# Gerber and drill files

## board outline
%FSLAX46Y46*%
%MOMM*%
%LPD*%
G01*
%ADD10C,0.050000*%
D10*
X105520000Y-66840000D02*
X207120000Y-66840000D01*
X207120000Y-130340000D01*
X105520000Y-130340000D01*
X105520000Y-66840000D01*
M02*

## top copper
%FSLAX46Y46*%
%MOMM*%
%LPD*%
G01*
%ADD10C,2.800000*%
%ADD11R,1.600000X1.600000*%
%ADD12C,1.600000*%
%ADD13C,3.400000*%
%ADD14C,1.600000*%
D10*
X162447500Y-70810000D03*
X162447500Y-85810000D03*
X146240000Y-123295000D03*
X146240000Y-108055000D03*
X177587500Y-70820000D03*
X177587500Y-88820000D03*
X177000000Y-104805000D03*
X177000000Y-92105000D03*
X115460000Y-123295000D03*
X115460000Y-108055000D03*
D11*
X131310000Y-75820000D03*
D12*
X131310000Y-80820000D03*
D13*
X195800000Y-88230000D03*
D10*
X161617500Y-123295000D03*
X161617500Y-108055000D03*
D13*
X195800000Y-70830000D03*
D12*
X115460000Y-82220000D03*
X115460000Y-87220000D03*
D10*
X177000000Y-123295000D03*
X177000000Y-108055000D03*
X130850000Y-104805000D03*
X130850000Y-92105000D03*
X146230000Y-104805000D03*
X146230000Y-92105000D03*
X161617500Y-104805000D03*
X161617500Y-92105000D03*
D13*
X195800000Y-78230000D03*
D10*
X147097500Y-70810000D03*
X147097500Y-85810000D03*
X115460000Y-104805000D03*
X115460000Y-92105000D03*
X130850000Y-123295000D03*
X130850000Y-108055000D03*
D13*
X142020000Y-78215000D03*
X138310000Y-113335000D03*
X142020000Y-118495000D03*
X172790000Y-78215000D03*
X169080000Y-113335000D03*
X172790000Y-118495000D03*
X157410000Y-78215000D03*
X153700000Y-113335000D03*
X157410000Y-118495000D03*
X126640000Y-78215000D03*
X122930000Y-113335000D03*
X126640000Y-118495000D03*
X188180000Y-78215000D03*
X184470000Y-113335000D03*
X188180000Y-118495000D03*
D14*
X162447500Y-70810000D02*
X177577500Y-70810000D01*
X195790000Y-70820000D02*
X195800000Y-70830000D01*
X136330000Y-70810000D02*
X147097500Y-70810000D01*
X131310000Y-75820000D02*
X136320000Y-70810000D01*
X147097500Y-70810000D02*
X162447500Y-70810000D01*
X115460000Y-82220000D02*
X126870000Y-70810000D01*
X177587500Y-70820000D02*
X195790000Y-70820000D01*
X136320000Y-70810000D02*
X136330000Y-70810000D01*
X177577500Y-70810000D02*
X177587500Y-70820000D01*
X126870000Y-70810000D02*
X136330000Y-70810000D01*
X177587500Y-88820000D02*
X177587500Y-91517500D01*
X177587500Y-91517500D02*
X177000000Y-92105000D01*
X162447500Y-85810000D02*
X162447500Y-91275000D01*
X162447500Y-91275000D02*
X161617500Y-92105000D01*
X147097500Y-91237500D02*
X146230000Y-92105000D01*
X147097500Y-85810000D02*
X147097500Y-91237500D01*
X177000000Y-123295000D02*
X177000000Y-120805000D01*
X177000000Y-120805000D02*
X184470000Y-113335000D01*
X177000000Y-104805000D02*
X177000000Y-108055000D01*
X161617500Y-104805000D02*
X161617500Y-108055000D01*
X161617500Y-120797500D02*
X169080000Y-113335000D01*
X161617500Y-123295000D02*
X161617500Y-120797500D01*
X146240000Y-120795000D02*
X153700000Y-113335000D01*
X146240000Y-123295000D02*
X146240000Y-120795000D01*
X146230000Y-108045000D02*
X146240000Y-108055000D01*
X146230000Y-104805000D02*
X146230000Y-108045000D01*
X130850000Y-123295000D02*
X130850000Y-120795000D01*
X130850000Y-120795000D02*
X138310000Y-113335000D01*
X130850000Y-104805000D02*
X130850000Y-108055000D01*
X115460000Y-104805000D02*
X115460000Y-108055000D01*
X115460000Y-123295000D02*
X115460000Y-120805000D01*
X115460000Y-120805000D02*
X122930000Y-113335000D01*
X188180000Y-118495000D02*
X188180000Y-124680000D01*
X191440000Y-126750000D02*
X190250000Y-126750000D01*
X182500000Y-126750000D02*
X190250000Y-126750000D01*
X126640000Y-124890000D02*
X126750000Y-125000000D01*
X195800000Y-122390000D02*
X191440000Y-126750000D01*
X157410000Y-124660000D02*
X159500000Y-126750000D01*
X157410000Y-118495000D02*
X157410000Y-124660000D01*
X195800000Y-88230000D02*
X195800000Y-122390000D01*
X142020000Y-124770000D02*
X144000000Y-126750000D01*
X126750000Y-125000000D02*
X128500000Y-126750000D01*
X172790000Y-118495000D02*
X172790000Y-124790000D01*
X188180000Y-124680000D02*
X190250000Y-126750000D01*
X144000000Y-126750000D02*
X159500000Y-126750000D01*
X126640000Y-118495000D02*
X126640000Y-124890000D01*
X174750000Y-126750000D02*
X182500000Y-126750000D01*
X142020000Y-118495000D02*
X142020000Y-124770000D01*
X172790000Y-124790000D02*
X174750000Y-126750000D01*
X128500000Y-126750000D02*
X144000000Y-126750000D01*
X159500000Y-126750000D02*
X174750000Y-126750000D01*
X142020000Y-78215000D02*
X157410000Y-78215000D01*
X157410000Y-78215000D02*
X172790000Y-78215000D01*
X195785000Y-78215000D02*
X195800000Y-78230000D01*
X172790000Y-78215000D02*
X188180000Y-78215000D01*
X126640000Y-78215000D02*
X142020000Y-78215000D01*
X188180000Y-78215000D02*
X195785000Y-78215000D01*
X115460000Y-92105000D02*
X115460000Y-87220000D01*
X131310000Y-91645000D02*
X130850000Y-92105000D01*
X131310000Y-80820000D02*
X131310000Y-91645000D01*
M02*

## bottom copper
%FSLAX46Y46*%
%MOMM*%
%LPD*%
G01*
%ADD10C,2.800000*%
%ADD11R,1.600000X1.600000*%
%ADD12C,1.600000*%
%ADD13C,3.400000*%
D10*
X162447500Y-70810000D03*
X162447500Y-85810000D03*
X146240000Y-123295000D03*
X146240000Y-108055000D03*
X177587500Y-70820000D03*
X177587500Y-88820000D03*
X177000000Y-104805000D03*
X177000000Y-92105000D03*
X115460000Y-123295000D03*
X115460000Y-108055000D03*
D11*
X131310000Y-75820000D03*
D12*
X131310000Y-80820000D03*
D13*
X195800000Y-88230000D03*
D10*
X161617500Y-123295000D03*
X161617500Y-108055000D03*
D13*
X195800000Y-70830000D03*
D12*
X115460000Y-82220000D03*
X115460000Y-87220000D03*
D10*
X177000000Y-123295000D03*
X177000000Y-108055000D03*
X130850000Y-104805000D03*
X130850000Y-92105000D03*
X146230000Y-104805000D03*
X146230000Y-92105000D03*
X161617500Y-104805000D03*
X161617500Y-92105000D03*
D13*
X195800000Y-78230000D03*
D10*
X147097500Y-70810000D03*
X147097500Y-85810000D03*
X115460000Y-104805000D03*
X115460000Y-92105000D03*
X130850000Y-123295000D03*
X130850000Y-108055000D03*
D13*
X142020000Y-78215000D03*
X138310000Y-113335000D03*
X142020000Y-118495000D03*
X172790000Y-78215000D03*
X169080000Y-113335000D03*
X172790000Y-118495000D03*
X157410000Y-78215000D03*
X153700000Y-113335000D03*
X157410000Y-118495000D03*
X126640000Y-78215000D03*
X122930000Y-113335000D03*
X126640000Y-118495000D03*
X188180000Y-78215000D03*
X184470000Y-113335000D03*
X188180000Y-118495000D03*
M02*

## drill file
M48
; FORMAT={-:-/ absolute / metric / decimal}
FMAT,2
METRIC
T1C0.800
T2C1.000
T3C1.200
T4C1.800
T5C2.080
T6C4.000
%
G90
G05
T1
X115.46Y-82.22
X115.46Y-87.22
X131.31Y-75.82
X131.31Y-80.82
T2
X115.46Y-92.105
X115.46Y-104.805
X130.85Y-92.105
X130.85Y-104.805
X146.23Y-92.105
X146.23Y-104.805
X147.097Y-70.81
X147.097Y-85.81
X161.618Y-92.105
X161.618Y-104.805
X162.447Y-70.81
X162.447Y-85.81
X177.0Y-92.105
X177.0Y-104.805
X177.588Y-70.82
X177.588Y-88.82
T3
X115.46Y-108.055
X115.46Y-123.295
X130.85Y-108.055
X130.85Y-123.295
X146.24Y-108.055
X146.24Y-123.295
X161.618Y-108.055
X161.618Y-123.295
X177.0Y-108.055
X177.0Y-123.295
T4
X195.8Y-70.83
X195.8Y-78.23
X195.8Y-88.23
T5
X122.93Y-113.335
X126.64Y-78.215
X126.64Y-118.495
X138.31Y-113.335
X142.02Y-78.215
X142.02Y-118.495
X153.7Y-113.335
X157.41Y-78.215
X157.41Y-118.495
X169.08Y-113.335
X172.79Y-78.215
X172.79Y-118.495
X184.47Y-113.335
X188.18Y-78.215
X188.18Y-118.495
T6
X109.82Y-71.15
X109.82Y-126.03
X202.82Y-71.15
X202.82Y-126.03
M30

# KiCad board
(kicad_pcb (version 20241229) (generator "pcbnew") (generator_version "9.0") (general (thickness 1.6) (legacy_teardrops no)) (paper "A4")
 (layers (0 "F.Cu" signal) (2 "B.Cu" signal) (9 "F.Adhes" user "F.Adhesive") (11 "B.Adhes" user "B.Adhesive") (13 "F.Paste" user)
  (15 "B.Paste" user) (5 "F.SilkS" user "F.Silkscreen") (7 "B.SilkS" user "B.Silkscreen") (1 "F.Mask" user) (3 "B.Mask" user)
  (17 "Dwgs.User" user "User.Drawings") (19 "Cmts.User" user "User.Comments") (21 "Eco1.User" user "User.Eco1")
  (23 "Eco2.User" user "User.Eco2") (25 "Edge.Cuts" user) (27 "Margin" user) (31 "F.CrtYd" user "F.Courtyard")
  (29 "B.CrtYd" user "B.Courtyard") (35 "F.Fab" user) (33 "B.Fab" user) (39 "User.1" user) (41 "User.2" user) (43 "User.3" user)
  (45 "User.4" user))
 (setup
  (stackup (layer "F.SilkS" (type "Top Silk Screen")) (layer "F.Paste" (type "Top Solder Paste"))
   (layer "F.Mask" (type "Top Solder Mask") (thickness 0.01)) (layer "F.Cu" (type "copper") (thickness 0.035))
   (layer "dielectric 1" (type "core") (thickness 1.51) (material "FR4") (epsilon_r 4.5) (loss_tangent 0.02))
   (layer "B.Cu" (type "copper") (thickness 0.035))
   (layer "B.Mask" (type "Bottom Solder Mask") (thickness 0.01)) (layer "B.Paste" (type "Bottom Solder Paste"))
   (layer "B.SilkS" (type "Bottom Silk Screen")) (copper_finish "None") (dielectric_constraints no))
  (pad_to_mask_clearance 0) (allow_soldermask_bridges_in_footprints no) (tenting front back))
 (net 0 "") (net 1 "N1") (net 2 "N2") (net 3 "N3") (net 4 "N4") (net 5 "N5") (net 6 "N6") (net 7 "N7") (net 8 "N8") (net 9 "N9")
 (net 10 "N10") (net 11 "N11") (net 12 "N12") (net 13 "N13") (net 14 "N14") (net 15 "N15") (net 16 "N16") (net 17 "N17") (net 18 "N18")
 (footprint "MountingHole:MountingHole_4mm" (layer "F.Cu") (at 202.82 126.03)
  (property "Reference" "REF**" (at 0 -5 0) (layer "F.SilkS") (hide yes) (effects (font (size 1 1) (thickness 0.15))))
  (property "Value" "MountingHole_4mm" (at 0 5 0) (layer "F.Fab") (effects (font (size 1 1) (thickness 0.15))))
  (pad "" np_thru_hole circle (at 0 0) (size 4 4) (drill 4) (layers "*.Cu" "*.Mask")))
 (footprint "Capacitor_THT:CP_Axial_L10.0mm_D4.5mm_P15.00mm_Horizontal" (layer "F.Cu") (at 162.4475 70.81 -90)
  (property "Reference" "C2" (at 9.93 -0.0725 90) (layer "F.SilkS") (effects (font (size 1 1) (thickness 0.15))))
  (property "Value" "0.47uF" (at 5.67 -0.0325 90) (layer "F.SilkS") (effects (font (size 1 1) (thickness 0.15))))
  (pad "1" thru_hole circle (at 0 0 270) (size 2.8 2.8) (drill 1) (layers "*.Cu" "*.Mask") (remove_unused_layers no) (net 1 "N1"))
  (pad "2" thru_hole circle (at 15 0 270) (size 2.8 2.8) (drill 1) (layers "*.Cu" "*.Mask") (remove_unused_layers no) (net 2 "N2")))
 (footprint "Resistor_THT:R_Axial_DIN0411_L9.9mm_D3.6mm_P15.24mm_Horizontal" (layer "F.Cu") (at 146.24 123.295 90)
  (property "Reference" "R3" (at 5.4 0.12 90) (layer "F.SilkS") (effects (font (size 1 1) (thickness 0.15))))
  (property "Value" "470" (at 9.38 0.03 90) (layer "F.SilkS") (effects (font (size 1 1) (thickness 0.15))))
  (pad "1" thru_hole circle (at 0 0 90) (size 2.8 2.8) (drill 1.2) (layers "*.Cu" "*.Mask") (remove_unused_layers no) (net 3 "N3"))
  (pad "2" thru_hole circle (at 15.24 0 90) (size 2.8 2.8) (drill 1.2) (layers "*.Cu" "*.Mask") (remove_unused_layers no) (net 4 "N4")))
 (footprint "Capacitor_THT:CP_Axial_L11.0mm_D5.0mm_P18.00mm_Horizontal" (layer "F.Cu") (at 177.5875 70.82 -90)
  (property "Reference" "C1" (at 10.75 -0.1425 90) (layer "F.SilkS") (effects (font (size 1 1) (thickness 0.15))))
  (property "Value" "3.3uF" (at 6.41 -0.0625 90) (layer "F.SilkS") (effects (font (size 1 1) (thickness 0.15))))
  (pad "1" thru_hole circle (at 0 0 270) (size 2.8 2.8) (drill 1) (layers "*.Cu" "*.Mask") (remove_unused_layers no) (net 1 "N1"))
  (pad "2" thru_hole circle (at 18 0 270) (size 2.8 2.8) (drill 1) (layers "*.Cu" "*.Mask") (remove_unused_layers no) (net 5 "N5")))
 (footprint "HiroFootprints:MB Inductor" (layer "F.Cu") (at 177 104.805 90)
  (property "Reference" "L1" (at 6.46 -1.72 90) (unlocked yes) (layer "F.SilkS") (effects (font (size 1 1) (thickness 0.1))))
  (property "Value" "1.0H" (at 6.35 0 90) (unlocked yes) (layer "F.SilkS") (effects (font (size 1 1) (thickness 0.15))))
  (pad "1" thru_hole circle (at 0 0 90) (size 2.8 2.8) (drill 1) (layers "*.Cu" "*.Mask") (remove_unused_layers no) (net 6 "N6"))
  (pad "2" thru_hole circle (at 12.7 0 90) (size 2.8 2.8) (drill 1) (layers "*.Cu" "*.Mask") (remove_unused_layers no) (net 5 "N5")))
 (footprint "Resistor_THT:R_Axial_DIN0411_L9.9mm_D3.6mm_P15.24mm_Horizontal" (layer "F.Cu") (at 115.46 123.295 90)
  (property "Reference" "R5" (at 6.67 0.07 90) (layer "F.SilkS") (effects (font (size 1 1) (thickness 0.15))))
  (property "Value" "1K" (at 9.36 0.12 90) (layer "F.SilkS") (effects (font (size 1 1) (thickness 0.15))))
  (pad "1" thru_hole circle (at 0 0 90) (size 2.8 2.8) (drill 1.2) (layers "*.Cu" "*.Mask") (remove_unused_layers no) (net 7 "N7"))
  (pad "2" thru_hole circle (at 15.24 0 90) (size 2.8 2.8) (drill 1.2) (layers "*.Cu" "*.Mask") (remove_unused_layers no) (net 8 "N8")))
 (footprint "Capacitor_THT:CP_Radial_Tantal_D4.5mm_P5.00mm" (layer "F.Cu") (at 131.31 75.82 -90)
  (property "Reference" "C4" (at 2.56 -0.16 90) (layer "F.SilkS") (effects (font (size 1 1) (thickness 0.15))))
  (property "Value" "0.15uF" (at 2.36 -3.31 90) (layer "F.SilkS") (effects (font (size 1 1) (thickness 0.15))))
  (pad "1" thru_hole rect (at 0 0 270) (size 1.6 1.6) (drill 0.8) (layers "*.Cu" "*.Mask") (remove_unused_layers no) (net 1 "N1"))
  (pad "2" thru_hole circle (at 5 0 270) (size 1.6 1.6) (drill 0.8) (layers "*.Cu" "*.Mask") (remove_unused_layers no) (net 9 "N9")))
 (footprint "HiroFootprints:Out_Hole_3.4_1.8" (layer "F.Cu") (at 195.8 88.23)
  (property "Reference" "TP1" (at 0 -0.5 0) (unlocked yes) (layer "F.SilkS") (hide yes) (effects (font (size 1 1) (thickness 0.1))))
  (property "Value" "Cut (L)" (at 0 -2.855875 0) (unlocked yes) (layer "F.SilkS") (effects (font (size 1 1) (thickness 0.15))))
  (pad "1" thru_hole circle (at 0 0) (size 3.4 3.4) (drill 1.8) (layers "*.Cu" "*.Mask") (remove_unused_layers no) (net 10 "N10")))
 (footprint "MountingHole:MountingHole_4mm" (layer "F.Cu") (at 109.82 71.15)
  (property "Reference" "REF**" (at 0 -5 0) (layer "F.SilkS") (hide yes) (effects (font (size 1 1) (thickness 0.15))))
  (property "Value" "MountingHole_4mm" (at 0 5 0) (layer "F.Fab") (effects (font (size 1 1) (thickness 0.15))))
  (pad "" np_thru_hole circle (at 0 0) (size 4 4) (drill 4) (layers "*.Cu" "*.Mask")))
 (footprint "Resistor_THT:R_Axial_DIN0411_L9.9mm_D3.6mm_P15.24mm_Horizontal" (layer "F.Cu") (at 161.6175 123.295 90)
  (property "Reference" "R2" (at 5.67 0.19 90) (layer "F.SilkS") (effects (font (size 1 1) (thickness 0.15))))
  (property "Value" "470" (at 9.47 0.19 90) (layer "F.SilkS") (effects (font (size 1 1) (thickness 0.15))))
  (pad "1" thru_hole circle (at 0 0 90) (size 2.8 2.8) (drill 1.2) (layers "*.Cu" "*.Mask") (remove_unused_layers no) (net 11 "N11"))
  (pad "2" thru_hole circle (at 15.24 0 90) (size 2.8 2.8) (drill 1.2) (layers "*.Cu" "*.Mask") (remove_unused_layers no) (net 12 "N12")))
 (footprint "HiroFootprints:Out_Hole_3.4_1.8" (layer "F.Cu") (at 195.8 70.83)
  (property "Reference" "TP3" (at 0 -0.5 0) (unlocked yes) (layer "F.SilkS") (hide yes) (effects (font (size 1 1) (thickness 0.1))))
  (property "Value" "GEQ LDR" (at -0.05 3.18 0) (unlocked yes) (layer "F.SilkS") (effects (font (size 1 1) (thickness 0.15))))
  (pad "1" thru_hole circle (at 0 0) (size 3.4 3.4) (drill 1.8) (layers "*.Cu" "*.Mask") (remove_unused_layers no) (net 1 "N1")))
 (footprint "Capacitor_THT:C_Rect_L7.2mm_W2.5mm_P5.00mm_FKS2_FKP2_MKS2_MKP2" (layer "F.Cu") (at 115.46 82.22 -90)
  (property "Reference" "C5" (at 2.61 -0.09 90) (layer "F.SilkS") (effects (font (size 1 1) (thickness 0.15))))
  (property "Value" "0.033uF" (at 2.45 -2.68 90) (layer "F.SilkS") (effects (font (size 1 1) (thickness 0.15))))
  (pad "1" thru_hole circle (at 0 0 270) (size 1.6 1.6) (drill 0.8) (layers "*.Cu" "*.Mask") (remove_unused_layers no) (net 1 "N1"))
  (pad "2" thru_hole circle (at 5 0 270) (size 1.6 1.6) (drill 0.8) (layers "*.Cu" "*.Mask") (remove_unused_layers no) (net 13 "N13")))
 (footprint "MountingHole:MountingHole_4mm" (layer "F.Cu") (at 202.82 71.15)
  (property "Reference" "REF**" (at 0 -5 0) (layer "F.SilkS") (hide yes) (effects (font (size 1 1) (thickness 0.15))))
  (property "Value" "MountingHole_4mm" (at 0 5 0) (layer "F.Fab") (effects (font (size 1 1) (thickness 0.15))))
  (pad "" np_thru_hole circle (at 0 0) (size 4 4) (drill 4) (layers "*.Cu" "*.Mask")))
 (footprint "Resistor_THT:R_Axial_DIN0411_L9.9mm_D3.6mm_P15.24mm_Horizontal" (layer "F.Cu") (at 177 123.295 90)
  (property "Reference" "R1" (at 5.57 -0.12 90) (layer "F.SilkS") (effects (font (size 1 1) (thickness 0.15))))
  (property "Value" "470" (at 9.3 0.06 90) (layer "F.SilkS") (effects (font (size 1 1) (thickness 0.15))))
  (pad "1" thru_hole circle (at 0 0 90) (size 2.8 2.8) (drill 1.2) (layers "*.Cu" "*.Mask") (remove_unused_layers no) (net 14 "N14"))
  (pad "2" thru_hole circle (at 15.24 0 90) (size 2.8 2.8) (drill 1.2) (layers "*.Cu" "*.Mask") (remove_unused_layers no) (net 6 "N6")))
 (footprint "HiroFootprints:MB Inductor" (layer "F.Cu") (at 130.85 104.805 90)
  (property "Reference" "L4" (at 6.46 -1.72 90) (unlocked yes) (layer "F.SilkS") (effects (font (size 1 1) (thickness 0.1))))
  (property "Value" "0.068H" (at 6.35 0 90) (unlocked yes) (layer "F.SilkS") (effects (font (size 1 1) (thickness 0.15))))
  (pad "1" thru_hole circle (at 0 0 90) (size 2.8 2.8) (drill 1) (layers "*.Cu" "*.Mask") (remove_unused_layers no) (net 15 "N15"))
  (pad "2" thru_hole circle (at 12.7 0 90) (size 2.8 2.8) (drill 1) (layers "*.Cu" "*.Mask") (remove_unused_layers no) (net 9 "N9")))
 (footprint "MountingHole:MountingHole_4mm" (layer "F.Cu") (at 109.82 126.03)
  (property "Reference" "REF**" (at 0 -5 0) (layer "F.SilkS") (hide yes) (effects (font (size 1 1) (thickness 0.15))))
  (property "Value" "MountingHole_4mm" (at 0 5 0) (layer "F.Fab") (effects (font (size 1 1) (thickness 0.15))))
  (pad "" np_thru_hole circle (at 0 0) (size 4 4) (drill 4) (layers "*.Cu" "*.Mask")))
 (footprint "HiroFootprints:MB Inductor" (layer "F.Cu") (at 146.23 104.805 90)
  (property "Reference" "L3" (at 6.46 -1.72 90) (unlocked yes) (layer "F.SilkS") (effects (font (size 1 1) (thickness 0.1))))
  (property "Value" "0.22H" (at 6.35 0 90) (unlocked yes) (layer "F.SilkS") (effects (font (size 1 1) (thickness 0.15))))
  (pad "1" thru_hole circle (at 0 0 90) (size 2.8 2.8) (drill 1) (layers "*.Cu" "*.Mask") (remove_unused_layers no) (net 4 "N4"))
  (pad "2" thru_hole circle (at 12.7 0 90) (size 2.8 2.8) (drill 1) (layers "*.Cu" "*.Mask") (remove_unused_layers no) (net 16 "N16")))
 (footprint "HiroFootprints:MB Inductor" (layer "F.Cu") (at 161.6175 104.805 90)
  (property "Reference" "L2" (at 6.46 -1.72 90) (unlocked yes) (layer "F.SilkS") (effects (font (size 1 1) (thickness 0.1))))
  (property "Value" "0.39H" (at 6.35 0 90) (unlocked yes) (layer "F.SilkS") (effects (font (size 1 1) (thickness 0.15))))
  (pad "1" thru_hole circle (at 0 0 90) (size 2.8 2.8) (drill 1) (layers "*.Cu" "*.Mask") (remove_unused_layers no) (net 12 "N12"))
  (pad "2" thru_hole circle (at 12.7 0 90) (size 2.8 2.8) (drill 1) (layers "*.Cu" "*.Mask") (remove_unused_layers no) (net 2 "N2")))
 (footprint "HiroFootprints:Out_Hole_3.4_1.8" (layer "F.Cu") (at 195.8 78.23)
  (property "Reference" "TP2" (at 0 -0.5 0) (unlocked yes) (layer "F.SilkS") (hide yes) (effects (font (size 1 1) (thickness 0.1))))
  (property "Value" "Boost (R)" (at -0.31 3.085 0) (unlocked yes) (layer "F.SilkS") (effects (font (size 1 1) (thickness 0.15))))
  (pad "1" thru_hole circle (at 0 0) (size 3.4 3.4) (drill 1.8) (layers "*.Cu" "*.Mask") (remove_unused_layers no) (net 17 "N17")))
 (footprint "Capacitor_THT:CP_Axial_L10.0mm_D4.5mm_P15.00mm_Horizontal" (layer "F.Cu") (at 147.0975 70.81 -90)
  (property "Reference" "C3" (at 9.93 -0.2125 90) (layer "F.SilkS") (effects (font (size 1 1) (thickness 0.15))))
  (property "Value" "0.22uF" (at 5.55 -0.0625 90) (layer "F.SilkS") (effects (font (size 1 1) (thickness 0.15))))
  (pad "1" thru_hole circle (at 0 0 270) (size 2.8 2.8) (drill 1) (layers "*.Cu" "*.Mask") (remove_unused_layers no) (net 1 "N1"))
  (pad "2" thru_hole circle (at 15 0 270) (size 2.8 2.8) (drill 1) (layers "*.Cu" "*.Mask") (remove_unused_layers no) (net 16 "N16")))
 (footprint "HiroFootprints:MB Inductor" (layer "F.Cu") (at 115.46 104.805 90)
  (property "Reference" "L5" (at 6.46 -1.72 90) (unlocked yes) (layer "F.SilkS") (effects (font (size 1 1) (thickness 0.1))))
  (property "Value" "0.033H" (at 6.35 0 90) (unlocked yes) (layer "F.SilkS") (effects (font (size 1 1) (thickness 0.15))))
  (pad "1" thru_hole circle (at 0 0 90) (size 2.8 2.8) (drill 1) (layers "*.Cu" "*.Mask") (remove_unused_layers no) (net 8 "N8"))
  (pad "2" thru_hole circle (at 12.7 0 90) (size 2.8 2.8) (drill 1) (layers "*.Cu" "*.Mask") (remove_unused_layers no) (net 13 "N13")))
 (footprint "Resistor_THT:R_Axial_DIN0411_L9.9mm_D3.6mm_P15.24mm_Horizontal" (layer "F.Cu") (at 130.85 123.295 90)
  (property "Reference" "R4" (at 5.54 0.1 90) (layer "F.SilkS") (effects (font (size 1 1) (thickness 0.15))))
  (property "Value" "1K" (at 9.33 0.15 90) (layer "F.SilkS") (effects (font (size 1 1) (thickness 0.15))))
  (pad "1" thru_hole circle (at 0 0 90) (size 2.8 2.8) (drill 1.2) (layers "*.Cu" "*.Mask") (remove_unused_layers no) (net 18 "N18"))
  (pad "2" thru_hole circle (at 15.24 0 90) (size 2.8 2.8) (drill 1.2) (layers "*.Cu" "*.Mask") (remove_unused_layers no) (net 15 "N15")))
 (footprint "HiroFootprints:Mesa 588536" (layer "B.Cu") (at 142.02 124.035 -90)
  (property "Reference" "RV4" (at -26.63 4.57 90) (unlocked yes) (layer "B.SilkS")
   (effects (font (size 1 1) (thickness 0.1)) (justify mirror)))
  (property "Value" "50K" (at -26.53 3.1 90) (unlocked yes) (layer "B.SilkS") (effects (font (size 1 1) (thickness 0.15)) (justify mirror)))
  (pad "1" thru_hole circle (at -45.82 0 270) (size 3.4 3.4) (drill 2.08) (layers "*.Cu" "*.Mask") (remove_unused_layers no) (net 17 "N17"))
  (pad "2" thru_hole circle (at -10.7 3.71 270) (size 3.4 3.4) (drill 2.08) (layers "*.Cu" "*.Mask") (remove_unused_layers no)
   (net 18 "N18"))
  (pad "3" thru_hole circle (at -5.54 0 270) (size 3.4 3.4) (drill 2.08) (layers "*.Cu" "*.Mask") (remove_unused_layers no) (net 10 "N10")))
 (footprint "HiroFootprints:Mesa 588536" (layer "B.Cu") (at 172.79 124.035 -90)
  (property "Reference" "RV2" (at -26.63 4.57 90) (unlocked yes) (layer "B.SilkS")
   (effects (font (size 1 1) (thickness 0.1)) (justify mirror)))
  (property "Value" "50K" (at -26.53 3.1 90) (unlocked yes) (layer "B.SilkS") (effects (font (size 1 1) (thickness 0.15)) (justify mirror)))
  (pad "1" thru_hole circle (at -45.82 0 270) (size 3.4 3.4) (drill 2.08) (layers "*.Cu" "*.Mask") (remove_unused_layers no) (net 17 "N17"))
  (pad "2" thru_hole circle (at -10.7 3.71 270) (size 3.4 3.4) (drill 2.08) (layers "*.Cu" "*.Mask") (remove_unused_layers no)
   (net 11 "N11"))
  (pad "3" thru_hole circle (at -5.54 0 270) (size 3.4 3.4) (drill 2.08) (layers "*.Cu" "*.Mask") (remove_unused_layers no) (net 10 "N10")))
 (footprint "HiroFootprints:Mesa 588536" (layer "B.Cu") (at 157.41 124.035 -90)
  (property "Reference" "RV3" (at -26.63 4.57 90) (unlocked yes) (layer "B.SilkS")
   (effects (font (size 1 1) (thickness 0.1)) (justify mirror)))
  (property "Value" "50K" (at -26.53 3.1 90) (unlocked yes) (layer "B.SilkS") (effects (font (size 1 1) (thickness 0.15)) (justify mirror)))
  (pad "1" thru_hole circle (at -45.82 0 270) (size 3.4 3.4) (drill 2.08) (layers "*.Cu" "*.Mask") (remove_unused_layers no) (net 17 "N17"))
  (pad "2" thru_hole circle (at -10.7 3.71 270) (size 3.4 3.4) (drill 2.08) (layers "*.Cu" "*.Mask") (remove_unused_layers no) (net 3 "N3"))
  (pad "3" thru_hole circle (at -5.54 0 270) (size 3.4 3.4) (drill 2.08) (layers "*.Cu" "*.Mask") (remove_unused_layers no) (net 10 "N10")))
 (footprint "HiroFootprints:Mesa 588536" (layer "B.Cu") (at 126.64 124.035 -90)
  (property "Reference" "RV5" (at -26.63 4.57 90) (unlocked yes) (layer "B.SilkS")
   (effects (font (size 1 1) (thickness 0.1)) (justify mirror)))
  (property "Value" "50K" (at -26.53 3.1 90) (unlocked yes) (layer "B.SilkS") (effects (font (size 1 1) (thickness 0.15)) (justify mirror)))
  (pad "1" thru_hole circle (at -45.82 0 270) (size 3.4 3.4) (drill 2.08) (layers "*.Cu" "*.Mask") (remove_unused_layers no) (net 17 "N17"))
  (pad "2" thru_hole circle (at -10.7 3.71 270) (size 3.4 3.4) (drill 2.08) (layers "*.Cu" "*.Mask") (remove_unused_layers no) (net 7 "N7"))
  (pad "3" thru_hole circle (at -5.54 0 270) (size 3.4 3.4) (drill 2.08) (layers "*.Cu" "*.Mask") (remove_unused_layers no) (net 10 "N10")))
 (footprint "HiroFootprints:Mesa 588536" (layer "B.Cu") (at 188.18 124.035 -90)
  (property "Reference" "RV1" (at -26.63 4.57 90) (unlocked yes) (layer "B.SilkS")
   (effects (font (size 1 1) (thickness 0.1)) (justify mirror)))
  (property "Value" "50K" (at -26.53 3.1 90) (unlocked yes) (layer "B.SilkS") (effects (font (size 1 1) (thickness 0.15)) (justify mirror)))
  (pad "1" thru_hole circle (at -45.82 0 270) (size 3.4 3.4) (drill 2.08) (layers "*.Cu" "*.Mask") (remove_unused_layers no) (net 17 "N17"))
  (pad "2" thru_hole circle (at -10.7 3.71 270) (size 3.4 3.4) (drill 2.08) (layers "*.Cu" "*.Mask") (remove_unused_layers no)
   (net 14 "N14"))
  (pad "3" thru_hole circle (at -5.54 0 270) (size 3.4 3.4) (drill 2.08) (layers "*.Cu" "*.Mask") (remove_unused_layers no) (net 10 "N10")))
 (gr_rect (start 105.52 66.84) (end 207.12 130.34) (stroke (width 0.05) (type solid)) (fill no) (layer "Edge.Cuts"))
 (segment (start 162.4475 70.81) (end 177.5775 70.81) (width 1.6) (layer "F.Cu") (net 1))
 (segment (start 195.79 70.82) (end 195.8 70.83) (width 1.6) (layer "F.Cu") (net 1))
 (segment (start 136.33 70.81) (end 147.0975 70.81) (width 1.6) (layer "F.Cu") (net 1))
 (segment (start 131.31 75.82) (end 136.32 70.81) (width 1.6) (layer "F.Cu") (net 1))
 (segment (start 147.0975 70.81) (end 162.4475 70.81) (width 1.6) (layer "F.Cu") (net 1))
 (segment (start 115.46 82.22) (end 126.87 70.81) (width 1.6) (layer "F.Cu") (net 1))
 (segment (start 177.5875 70.82) (end 195.79 70.82) (width 1.6) (layer "F.Cu") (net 1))
 (segment (start 136.32 70.81) (end 136.33 70.81) (width 1.6) (layer "F.Cu") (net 1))
 (segment (start 177.5775 70.81) (end 177.5875 70.82) (width 1.6) (layer "F.Cu") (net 1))
 (segment (start 126.87 70.81) (end 136.33 70.81) (width 1.6) (layer "F.Cu") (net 1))
 (segment (start 177.5875 88.82) (end 177.5875 91.5175) (width 1.6) (layer "F.Cu") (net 5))
 (segment (start 177.5875 91.5175) (end 177 92.105) (width 1.6) (layer "F.Cu") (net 5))
 (segment (start 162.4475 85.81) (end 162.4475 91.275) (width 1.6) (layer "F.Cu") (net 2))
 (segment (start 162.4475 91.275) (end 161.6175 92.105) (width 1.6) (layer "F.Cu") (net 2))
 (segment (start 147.0975 91.2375) (end 146.23 92.105) (width 1.6) (layer "F.Cu") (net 16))
 (segment (start 147.0975 85.81) (end 147.0975 91.2375) (width 1.6) (layer "F.Cu") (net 16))
 (segment (start 177 123.295) (end 177 120.805) (width 1.6) (layer "F.Cu") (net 14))
 (segment (start 177 120.805) (end 184.47 113.335) (width 1.6) (layer "F.Cu") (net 14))
 (segment (start 177 104.805) (end 177 108.055) (width 1.6) (layer "F.Cu") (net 6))
 (segment (start 161.6175 104.805) (end 161.6175 108.055) (width 1.6) (layer "F.Cu") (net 12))
 (segment (start 161.6175 120.7975) (end 169.08 113.335) (width 1.6) (layer "F.Cu") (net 11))
 (segment (start 161.6175 123.295) (end 161.6175 120.7975) (width 1.6) (layer "F.Cu") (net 11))
 (segment (start 146.24 120.795) (end 153.7 113.335) (width 1.6) (layer "F.Cu") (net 3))
 (segment (start 146.24 123.295) (end 146.24 120.795) (width 1.6) (layer "F.Cu") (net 3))
 (segment (start 146.23 108.045) (end 146.24 108.055) (width 1.6) (layer "F.Cu") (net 4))
 (segment (start 146.23 104.805) (end 146.23 108.045) (width 1.6) (layer "F.Cu") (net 4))
 (segment (start 130.85 123.295) (end 130.85 120.795) (width 1.6) (layer "F.Cu") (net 18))
 (segment (start 130.85 120.795) (end 138.31 113.335) (width 1.6) (layer "F.Cu") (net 18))
 (segment (start 130.85 104.805) (end 130.85 108.055) (width 1.6) (layer "F.Cu") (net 15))
 (segment (start 115.46 104.805) (end 115.46 108.055) (width 1.6) (layer "F.Cu") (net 8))
 (segment (start 115.46 123.295) (end 115.46 120.805) (width 1.6) (layer "F.Cu") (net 7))
 (segment (start 115.46 120.805) (end 122.93 113.335) (width 1.6) (layer "F.Cu") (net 7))
 (segment (start 188.18 118.495) (end 188.18 124.68) (width 1.6) (layer "F.Cu") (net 10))
 (segment (start 191.44 126.75) (end 190.25 126.75) (width 1.6) (layer "F.Cu") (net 10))
 (segment (start 182.5 126.75) (end 190.25 126.75) (width 1.6) (layer "F.Cu") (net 10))
 (segment (start 126.64 124.89) (end 126.75 125) (width 1.6) (layer "F.Cu") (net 10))
 (segment (start 195.8 122.39) (end 191.44 126.75) (width 1.6) (layer "F.Cu") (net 10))
 (segment (start 157.41 124.66) (end 159.5 126.75) (width 1.6) (layer "F.Cu") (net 10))
 (segment (start 157.41 118.495) (end 157.41 124.66) (width 1.6) (layer "F.Cu") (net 10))
 (segment (start 195.8 88.23) (end 195.8 122.39) (width 1.6) (layer "F.Cu") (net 10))
 (segment (start 142.02 124.77) (end 144 126.75) (width 1.6) (layer "F.Cu") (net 10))
 (segment (start 126.75 125) (end 128.5 126.75) (width 1.6) (layer "F.Cu") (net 10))
 (segment (start 172.79 118.495) (end 172.79 124.79) (width 1.6) (layer "F.Cu") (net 10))
 (segment (start 188.18 124.68) (end 190.25 126.75) (width 1.6) (layer "F.Cu") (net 10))
 (segment (start 144 126.75) (end 159.5 126.75) (width 1.6) (layer "F.Cu") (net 10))
 (segment (start 126.64 118.495) (end 126.64 124.89) (width 1.6) (layer "F.Cu") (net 10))
 (segment (start 174.75 126.75) (end 182.5 126.75) (width 1.6) (layer "F.Cu") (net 10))
 (segment (start 142.02 118.495) (end 142.02 124.77) (width 1.6) (layer "F.Cu") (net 10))
 (segment (start 172.79 124.79) (end 174.75 126.75) (width 1.6) (layer "F.Cu") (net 10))
 (segment (start 128.5 126.75) (end 144 126.75) (width 1.6) (layer "F.Cu") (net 10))
 (segment (start 159.5 126.75) (end 174.75 126.75) (width 1.6) (layer "F.Cu") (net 10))
 (segment (start 142.02 78.215) (end 157.41 78.215) (width 1.6) (layer "F.Cu") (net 17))
 (segment (start 157.41 78.215) (end 172.79 78.215) (width 1.6) (layer "F.Cu") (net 17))
 (segment (start 195.785 78.215) (end 195.8 78.23) (width 1.6) (layer "F.Cu") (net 17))
 (segment (start 172.79 78.215) (end 188.18 78.215) (width 1.6) (layer "F.Cu") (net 17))
 (segment (start 126.64 78.215) (end 142.02 78.215) (width 1.6) (layer "F.Cu") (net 17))
 (segment (start 188.18 78.215) (end 195.785 78.215) (width 1.6) (layer "F.Cu") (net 17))
 (segment (start 115.46 92.105) (end 115.46 87.22) (width 1.6) (layer "F.Cu") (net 13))
 (segment (start 131.31 91.645) (end 130.85 92.105) (width 1.6) (layer "F.Cu") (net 9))
 (segment (start 131.31 80.82) (end 131.31 91.645) (width 1.6) (layer "F.Cu") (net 9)))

